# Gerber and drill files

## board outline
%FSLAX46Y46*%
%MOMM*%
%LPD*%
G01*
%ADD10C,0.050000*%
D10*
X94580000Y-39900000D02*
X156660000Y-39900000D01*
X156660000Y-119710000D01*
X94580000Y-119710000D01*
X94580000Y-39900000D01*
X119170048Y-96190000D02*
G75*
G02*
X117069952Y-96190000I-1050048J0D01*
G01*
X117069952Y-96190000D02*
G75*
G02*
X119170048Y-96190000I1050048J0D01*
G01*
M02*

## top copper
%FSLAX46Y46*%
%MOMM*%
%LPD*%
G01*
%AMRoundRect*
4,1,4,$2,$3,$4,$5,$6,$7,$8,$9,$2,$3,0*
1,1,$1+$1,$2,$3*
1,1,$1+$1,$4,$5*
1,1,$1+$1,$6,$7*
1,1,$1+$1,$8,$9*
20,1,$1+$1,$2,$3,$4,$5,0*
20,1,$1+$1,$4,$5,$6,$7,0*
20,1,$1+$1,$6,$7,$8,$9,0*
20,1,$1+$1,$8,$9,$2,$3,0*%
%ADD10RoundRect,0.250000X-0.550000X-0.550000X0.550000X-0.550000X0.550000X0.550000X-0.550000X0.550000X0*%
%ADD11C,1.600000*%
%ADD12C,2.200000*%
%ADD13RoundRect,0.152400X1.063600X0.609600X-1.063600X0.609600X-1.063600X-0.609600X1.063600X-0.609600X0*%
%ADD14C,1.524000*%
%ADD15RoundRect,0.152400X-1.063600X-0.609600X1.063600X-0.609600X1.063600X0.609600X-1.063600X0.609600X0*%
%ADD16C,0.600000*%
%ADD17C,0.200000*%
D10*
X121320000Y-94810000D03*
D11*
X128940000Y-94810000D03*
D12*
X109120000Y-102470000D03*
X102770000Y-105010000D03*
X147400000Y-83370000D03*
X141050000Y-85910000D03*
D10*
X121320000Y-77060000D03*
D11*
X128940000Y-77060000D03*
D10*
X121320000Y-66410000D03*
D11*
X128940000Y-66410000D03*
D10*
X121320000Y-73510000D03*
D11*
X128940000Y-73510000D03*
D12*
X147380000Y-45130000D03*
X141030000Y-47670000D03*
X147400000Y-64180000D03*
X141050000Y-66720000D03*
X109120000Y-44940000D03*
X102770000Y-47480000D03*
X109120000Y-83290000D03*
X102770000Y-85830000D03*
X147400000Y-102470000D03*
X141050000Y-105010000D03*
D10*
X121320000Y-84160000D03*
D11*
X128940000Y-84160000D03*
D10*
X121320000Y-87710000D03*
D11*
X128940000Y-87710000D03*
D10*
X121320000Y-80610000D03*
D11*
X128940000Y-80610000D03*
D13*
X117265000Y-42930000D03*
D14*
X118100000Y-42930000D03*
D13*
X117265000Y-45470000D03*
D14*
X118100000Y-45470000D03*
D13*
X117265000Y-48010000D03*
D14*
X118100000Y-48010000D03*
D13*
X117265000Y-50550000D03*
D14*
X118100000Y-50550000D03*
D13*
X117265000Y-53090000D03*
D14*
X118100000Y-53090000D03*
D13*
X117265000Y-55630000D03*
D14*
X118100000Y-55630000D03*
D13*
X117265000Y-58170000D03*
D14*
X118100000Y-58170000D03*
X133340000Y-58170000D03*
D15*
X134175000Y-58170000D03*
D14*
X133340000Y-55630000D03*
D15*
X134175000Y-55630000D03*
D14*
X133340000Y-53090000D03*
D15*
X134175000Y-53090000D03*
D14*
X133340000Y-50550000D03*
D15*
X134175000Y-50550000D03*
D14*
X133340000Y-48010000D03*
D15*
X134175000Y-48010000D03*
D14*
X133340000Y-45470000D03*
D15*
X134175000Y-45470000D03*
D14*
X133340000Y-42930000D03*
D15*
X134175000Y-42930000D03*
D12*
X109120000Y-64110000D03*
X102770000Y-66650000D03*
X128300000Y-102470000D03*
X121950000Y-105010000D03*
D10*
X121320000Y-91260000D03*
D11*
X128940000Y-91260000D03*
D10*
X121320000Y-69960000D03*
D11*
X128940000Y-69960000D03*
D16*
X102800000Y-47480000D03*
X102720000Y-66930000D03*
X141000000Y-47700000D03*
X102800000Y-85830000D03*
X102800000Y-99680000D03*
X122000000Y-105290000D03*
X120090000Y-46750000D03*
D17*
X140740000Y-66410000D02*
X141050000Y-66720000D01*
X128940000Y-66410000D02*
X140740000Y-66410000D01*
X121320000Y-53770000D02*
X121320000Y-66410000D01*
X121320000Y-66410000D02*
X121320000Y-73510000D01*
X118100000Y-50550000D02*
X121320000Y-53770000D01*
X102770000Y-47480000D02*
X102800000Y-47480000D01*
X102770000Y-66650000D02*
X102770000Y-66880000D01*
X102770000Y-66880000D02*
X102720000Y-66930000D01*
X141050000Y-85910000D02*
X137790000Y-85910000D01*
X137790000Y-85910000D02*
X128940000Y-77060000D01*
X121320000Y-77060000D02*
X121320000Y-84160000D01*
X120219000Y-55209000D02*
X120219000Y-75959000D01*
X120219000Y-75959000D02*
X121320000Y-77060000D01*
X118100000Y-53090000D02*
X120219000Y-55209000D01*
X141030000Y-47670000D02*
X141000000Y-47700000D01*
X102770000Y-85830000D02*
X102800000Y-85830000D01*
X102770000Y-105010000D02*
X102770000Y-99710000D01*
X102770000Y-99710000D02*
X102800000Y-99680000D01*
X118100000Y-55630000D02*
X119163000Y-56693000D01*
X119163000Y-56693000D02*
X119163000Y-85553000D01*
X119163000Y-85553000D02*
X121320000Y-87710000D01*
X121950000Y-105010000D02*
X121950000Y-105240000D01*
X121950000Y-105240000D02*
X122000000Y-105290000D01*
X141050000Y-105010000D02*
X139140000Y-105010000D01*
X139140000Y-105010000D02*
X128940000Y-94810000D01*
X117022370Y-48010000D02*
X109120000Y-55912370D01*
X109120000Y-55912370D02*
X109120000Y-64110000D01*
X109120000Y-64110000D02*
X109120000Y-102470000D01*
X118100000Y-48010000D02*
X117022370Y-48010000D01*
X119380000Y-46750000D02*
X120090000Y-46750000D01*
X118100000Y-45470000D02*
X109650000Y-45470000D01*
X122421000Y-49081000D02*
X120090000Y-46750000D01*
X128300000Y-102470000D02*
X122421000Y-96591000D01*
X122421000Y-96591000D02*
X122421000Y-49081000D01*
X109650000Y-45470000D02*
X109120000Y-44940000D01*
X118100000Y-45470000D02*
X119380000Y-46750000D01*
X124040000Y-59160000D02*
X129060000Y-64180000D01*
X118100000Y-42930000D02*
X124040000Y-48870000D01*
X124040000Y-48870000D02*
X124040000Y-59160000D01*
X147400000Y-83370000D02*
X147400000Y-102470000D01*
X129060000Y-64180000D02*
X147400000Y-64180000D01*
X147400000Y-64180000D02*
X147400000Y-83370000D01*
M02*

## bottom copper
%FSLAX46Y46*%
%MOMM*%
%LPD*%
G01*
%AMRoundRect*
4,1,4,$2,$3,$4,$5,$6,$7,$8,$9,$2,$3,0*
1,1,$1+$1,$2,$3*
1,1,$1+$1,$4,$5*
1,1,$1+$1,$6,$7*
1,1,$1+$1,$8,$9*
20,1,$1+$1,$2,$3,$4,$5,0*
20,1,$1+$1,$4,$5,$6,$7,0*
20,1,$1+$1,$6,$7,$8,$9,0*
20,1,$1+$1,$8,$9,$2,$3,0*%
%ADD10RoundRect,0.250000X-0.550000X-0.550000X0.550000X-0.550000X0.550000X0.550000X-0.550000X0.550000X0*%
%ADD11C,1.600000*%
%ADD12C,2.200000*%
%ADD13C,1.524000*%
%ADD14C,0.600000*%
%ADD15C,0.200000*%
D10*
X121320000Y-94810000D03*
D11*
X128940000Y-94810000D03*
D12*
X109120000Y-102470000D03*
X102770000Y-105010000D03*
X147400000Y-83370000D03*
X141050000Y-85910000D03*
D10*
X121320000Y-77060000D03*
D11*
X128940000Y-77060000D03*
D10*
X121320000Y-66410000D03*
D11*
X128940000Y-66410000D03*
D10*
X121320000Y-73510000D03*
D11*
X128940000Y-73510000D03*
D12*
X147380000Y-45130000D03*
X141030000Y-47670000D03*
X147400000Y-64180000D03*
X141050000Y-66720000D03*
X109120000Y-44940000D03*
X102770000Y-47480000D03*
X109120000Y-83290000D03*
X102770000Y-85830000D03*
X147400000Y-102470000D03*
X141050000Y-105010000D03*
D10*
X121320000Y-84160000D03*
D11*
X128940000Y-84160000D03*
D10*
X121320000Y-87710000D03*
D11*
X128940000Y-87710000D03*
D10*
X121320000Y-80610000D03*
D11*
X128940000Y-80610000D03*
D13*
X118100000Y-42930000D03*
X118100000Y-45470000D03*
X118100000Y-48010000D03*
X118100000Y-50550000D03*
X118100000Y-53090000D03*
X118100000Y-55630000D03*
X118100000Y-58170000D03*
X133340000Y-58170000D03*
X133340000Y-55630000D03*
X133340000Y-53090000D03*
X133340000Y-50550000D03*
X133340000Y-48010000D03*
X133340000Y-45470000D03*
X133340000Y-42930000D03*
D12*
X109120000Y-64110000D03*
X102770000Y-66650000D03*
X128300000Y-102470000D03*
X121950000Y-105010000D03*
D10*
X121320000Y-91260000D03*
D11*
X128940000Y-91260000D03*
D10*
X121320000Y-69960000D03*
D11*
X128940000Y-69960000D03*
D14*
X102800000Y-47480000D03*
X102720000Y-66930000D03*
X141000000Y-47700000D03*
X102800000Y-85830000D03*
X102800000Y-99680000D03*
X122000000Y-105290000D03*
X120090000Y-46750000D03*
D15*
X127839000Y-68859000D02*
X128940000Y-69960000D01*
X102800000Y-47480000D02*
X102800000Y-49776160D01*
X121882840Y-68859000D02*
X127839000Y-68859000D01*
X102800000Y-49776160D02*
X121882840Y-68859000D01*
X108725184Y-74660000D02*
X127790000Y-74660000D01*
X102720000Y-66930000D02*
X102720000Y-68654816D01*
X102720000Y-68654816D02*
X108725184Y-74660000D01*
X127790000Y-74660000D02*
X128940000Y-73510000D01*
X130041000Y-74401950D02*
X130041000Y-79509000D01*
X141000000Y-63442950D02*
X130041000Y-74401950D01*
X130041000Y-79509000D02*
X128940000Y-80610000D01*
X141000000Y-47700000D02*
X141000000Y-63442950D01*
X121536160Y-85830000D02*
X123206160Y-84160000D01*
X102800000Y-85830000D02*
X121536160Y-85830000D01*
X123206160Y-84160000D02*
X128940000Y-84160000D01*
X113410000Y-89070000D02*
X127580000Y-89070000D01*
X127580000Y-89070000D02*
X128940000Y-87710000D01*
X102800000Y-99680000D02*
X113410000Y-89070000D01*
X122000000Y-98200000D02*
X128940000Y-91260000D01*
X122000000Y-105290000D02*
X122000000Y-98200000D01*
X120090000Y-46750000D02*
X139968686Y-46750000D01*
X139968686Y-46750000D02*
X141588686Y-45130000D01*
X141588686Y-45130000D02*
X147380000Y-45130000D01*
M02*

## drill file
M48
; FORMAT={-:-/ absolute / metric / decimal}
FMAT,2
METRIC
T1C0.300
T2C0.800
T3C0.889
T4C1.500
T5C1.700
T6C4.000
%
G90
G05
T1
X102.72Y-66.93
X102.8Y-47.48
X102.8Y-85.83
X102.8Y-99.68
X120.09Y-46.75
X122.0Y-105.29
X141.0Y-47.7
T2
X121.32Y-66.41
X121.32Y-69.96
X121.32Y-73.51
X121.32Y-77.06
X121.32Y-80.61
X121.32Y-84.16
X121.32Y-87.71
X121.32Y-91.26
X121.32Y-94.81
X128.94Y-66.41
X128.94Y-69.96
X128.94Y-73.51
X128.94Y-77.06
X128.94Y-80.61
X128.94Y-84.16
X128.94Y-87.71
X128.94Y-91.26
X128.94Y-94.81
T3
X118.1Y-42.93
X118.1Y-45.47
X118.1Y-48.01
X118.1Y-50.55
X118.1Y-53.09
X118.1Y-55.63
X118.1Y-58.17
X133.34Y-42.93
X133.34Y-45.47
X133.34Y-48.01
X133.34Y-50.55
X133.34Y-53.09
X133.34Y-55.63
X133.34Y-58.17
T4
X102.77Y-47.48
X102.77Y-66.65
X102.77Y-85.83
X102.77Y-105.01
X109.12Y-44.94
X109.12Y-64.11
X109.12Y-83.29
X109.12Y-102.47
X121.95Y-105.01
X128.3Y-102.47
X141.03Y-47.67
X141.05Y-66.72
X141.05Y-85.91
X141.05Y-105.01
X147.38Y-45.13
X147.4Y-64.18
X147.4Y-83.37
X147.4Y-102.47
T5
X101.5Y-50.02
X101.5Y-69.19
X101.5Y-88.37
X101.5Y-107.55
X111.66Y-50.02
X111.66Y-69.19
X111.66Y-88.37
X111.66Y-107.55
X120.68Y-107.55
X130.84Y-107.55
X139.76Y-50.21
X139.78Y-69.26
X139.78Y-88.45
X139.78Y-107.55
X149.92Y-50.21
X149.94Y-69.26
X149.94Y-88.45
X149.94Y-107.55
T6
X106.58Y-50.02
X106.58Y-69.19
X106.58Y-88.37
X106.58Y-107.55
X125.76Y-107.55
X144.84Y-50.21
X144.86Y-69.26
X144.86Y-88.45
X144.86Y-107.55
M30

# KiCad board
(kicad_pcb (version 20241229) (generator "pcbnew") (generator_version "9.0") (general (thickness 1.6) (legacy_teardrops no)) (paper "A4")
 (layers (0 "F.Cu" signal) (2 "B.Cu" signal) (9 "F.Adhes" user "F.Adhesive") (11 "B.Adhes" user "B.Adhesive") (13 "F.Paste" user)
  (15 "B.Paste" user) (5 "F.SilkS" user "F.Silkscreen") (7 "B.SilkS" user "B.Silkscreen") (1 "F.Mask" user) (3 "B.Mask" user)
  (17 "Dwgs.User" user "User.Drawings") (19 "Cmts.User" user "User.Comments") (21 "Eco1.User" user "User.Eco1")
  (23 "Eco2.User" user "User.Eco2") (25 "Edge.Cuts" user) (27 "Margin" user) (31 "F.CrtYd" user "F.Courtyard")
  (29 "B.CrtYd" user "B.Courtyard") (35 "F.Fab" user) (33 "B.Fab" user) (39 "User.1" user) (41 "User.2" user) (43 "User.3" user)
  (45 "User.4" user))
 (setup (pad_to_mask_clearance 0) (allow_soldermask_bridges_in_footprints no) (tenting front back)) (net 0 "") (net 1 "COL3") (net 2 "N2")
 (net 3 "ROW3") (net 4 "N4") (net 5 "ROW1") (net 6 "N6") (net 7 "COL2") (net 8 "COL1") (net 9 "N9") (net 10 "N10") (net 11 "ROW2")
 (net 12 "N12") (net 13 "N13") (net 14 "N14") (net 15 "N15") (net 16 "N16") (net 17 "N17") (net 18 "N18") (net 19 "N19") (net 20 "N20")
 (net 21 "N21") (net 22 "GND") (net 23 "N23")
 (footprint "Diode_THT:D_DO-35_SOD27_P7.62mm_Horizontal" (layer "F.Cu") (at 121.32 94.81)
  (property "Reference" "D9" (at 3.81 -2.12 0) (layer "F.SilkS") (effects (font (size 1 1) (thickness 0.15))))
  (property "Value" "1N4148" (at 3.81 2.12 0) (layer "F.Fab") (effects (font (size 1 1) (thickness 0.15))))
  (pad "1" thru_hole roundrect (at 0 0) (size 1.6 1.6) (drill 0.8) (layers "*.Cu" "*.Mask") (remove_unused_layers no)
   (roundrect_rratio 0.15625) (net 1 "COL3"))
  (pad "2" thru_hole circle (at 7.62 0) (size 1.6 1.6) (drill 0.8) (layers "*.Cu" "*.Mask") (remove_unused_layers no) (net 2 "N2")))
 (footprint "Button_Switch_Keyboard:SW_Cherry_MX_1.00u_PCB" (layer "F.Cu") (at 109.12 102.47)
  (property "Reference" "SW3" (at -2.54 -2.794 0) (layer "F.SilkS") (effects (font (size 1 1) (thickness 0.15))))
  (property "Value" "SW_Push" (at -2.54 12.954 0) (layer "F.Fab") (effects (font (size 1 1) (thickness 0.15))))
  (pad "" np_thru_hole circle (at -7.62 5.08) (size 1.7 1.7) (drill 1.7) (layers "*.Cu" "*.Mask"))
  (pad "" np_thru_hole circle (at -2.54 5.08) (size 4 4) (drill 4) (layers "*.Cu" "*.Mask"))
  (pad "" np_thru_hole circle (at 2.54 5.08) (size 1.7 1.7) (drill 1.7) (layers "*.Cu" "*.Mask"))
  (pad "1" thru_hole circle (at 0 0) (size 2.2 2.2) (drill 1.5) (layers "*.Cu" "*.Mask") (remove_unused_layers no) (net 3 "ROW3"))
  (pad "2" thru_hole circle (at -6.35 2.54) (size 2.2 2.2) (drill 1.5) (layers "*.Cu" "*.Mask") (remove_unused_layers no) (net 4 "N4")))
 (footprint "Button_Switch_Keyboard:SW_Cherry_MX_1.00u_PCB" (layer "F.Cu") (at 147.4 83.37)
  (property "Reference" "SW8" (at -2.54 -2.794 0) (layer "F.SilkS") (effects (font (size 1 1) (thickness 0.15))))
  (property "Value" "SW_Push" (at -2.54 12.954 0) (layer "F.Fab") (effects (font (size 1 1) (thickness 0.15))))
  (pad "" np_thru_hole circle (at -7.62 5.08) (size 1.7 1.7) (drill 1.7) (layers "*.Cu" "*.Mask"))
  (pad "" np_thru_hole circle (at -2.54 5.08) (size 4 4) (drill 4) (layers "*.Cu" "*.Mask"))
  (pad "" np_thru_hole circle (at 2.54 5.08) (size 1.7 1.7) (drill 1.7) (layers "*.Cu" "*.Mask"))
  (pad "1" thru_hole circle (at 0 0) (size 2.2 2.2) (drill 1.5) (layers "*.Cu" "*.Mask") (remove_unused_layers no) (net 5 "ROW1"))
  (pad "2" thru_hole circle (at -6.35 2.54) (size 2.2 2.2) (drill 1.5) (layers "*.Cu" "*.Mask") (remove_unused_layers no) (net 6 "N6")))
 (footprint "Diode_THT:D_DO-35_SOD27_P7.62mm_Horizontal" (layer "F.Cu") (at 121.32 77.06)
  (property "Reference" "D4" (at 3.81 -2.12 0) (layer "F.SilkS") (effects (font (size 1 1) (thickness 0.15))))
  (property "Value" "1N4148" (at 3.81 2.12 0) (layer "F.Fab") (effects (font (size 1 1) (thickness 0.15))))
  (pad "1" thru_hole roundrect (at 0 0) (size 1.6 1.6) (drill 0.8) (layers "*.Cu" "*.Mask") (remove_unused_layers no)
   (roundrect_rratio 0.15625) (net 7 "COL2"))
  (pad "2" thru_hole circle (at 7.62 0) (size 1.6 1.6) (drill 0.8) (layers "*.Cu" "*.Mask") (remove_unused_layers no) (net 6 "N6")))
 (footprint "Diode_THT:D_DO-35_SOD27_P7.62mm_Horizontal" (layer "F.Cu") (at 121.32 66.41)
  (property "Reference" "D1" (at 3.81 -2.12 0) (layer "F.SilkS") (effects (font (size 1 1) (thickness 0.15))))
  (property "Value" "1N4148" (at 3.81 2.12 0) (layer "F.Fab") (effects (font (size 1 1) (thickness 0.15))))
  (pad "1" thru_hole roundrect (at 0 0) (size 1.6 1.6) (drill 0.8) (layers "*.Cu" "*.Mask") (remove_unused_layers no)
   (roundrect_rratio 0.15625) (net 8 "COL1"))
  (pad "2" thru_hole circle (at 7.62 0) (size 1.6 1.6) (drill 0.8) (layers "*.Cu" "*.Mask") (remove_unused_layers no) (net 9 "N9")))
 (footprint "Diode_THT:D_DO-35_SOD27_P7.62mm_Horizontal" (layer "F.Cu") (at 121.32 73.51)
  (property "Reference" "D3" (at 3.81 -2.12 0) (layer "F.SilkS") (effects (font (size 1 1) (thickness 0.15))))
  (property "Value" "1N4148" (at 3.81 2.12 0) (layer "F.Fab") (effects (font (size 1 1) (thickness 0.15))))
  (pad "1" thru_hole roundrect (at 0 0) (size 1.6 1.6) (drill 0.8) (layers "*.Cu" "*.Mask") (remove_unused_layers no)
   (roundrect_rratio 0.15625) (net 8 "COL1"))
  (pad "2" thru_hole circle (at 7.62 0) (size 1.6 1.6) (drill 0.8) (layers "*.Cu" "*.Mask") (remove_unused_layers no) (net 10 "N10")))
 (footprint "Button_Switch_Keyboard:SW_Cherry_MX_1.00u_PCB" (layer "F.Cu") (at 147.38 45.13)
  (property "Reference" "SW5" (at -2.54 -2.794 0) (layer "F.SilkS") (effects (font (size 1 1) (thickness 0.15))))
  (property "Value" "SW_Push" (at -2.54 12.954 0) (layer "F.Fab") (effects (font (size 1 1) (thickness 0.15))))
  (pad "" np_thru_hole circle (at -7.62 5.08) (size 1.7 1.7) (drill 1.7) (layers "*.Cu" "*.Mask"))
  (pad "" np_thru_hole circle (at -2.54 5.08) (size 4 4) (drill 4) (layers "*.Cu" "*.Mask"))
  (pad "" np_thru_hole circle (at 2.54 5.08) (size 1.7 1.7) (drill 1.7) (layers "*.Cu" "*.Mask"))
  (pad "1" thru_hole circle (at 0 0) (size 2.2 2.2) (drill 1.5) (layers "*.Cu" "*.Mask") (remove_unused_layers no) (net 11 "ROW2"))
  (pad "2" thru_hole circle (at -6.35 2.54) (size 2.2 2.2) (drill 1.5) (layers "*.Cu" "*.Mask") (remove_unused_layers no) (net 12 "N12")))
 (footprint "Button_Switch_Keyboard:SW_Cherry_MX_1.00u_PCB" (layer "F.Cu") (at 147.4 64.18)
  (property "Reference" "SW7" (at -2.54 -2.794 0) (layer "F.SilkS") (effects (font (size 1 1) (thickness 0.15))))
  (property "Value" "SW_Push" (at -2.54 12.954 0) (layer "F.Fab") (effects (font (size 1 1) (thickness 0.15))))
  (pad "" np_thru_hole circle (at -7.62 5.08) (size 1.7 1.7) (drill 1.7) (layers "*.Cu" "*.Mask"))
  (pad "" np_thru_hole circle (at -2.54 5.08) (size 4 4) (drill 4) (layers "*.Cu" "*.Mask"))
  (pad "" np_thru_hole circle (at 2.54 5.08) (size 1.7 1.7) (drill 1.7) (layers "*.Cu" "*.Mask"))
  (pad "1" thru_hole circle (at 0 0) (size 2.2 2.2) (drill 1.5) (layers "*.Cu" "*.Mask") (remove_unused_layers no) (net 5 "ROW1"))
  (pad "2" thru_hole circle (at -6.35 2.54) (size 2.2 2.2) (drill 1.5) (layers "*.Cu" "*.Mask") (remove_unused_layers no) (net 9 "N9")))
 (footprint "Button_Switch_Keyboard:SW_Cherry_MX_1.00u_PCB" (layer "F.Cu") (at 109.12 44.94)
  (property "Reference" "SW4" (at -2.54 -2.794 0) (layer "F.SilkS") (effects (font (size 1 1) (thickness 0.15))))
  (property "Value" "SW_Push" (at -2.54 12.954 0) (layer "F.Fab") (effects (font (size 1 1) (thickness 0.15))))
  (pad "" np_thru_hole circle (at -7.62 5.08) (size 1.7 1.7) (drill 1.7) (layers "*.Cu" "*.Mask"))
  (pad "" np_thru_hole circle (at -2.54 5.08) (size 4 4) (drill 4) (layers "*.Cu" "*.Mask"))
  (pad "" np_thru_hole circle (at 2.54 5.08) (size 1.7 1.7) (drill 1.7) (layers "*.Cu" "*.Mask"))
  (pad "1" thru_hole circle (at 0 0) (size 2.2 2.2) (drill 1.5) (layers "*.Cu" "*.Mask") (remove_unused_layers no) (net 11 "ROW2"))
  (pad "2" thru_hole circle (at -6.35 2.54) (size 2.2 2.2) (drill 1.5) (layers "*.Cu" "*.Mask") (remove_unused_layers no) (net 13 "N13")))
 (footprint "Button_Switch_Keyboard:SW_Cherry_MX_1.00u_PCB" (layer "F.Cu") (at 109.12 83.29)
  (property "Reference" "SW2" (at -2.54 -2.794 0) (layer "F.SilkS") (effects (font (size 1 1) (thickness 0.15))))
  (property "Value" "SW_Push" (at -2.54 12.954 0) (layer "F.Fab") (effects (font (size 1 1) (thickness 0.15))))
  (pad "" np_thru_hole circle (at -7.62 5.08) (size 1.7 1.7) (drill 1.7) (layers "*.Cu" "*.Mask"))
  (pad "" np_thru_hole circle (at -2.54 5.08) (size 4 4) (drill 4) (layers "*.Cu" "*.Mask"))
  (pad "" np_thru_hole circle (at 2.54 5.08) (size 1.7 1.7) (drill 1.7) (layers "*.Cu" "*.Mask"))
  (pad "1" thru_hole circle (at 0 0) (size 2.2 2.2) (drill 1.5) (layers "*.Cu" "*.Mask") (remove_unused_layers no) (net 3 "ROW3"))
  (pad "2" thru_hole circle (at -6.35 2.54) (size 2.2 2.2) (drill 1.5) (layers "*.Cu" "*.Mask") (remove_unused_layers no) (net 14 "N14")))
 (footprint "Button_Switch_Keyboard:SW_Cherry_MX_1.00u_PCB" (layer "F.Cu") (at 147.4 102.47)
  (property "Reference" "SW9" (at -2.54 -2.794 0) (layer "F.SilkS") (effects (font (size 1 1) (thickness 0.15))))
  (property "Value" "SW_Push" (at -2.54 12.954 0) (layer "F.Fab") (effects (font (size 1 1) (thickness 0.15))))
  (pad "" np_thru_hole circle (at -7.62 5.08) (size 1.7 1.7) (drill 1.7) (layers "*.Cu" "*.Mask"))
  (pad "" np_thru_hole circle (at -2.54 5.08) (size 4 4) (drill 4) (layers "*.Cu" "*.Mask"))
  (pad "" np_thru_hole circle (at 2.54 5.08) (size 1.7 1.7) (drill 1.7) (layers "*.Cu" "*.Mask"))
  (pad "1" thru_hole circle (at 0 0) (size 2.2 2.2) (drill 1.5) (layers "*.Cu" "*.Mask") (remove_unused_layers no) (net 5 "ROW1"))
  (pad "2" thru_hole circle (at -6.35 2.54) (size 2.2 2.2) (drill 1.5) (layers "*.Cu" "*.Mask") (remove_unused_layers no) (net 2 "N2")))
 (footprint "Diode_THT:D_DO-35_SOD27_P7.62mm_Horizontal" (layer "F.Cu") (at 121.32 84.16)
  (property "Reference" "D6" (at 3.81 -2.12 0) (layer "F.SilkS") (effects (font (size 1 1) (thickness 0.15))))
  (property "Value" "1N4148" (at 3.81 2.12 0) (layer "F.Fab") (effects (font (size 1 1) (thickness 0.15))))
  (pad "1" thru_hole roundrect (at 0 0) (size 1.6 1.6) (drill 0.8) (layers "*.Cu" "*.Mask") (remove_unused_layers no)
   (roundrect_rratio 0.15625) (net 7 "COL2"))
  (pad "2" thru_hole circle (at 7.62 0) (size 1.6 1.6) (drill 0.8) (layers "*.Cu" "*.Mask") (remove_unused_layers no) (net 14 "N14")))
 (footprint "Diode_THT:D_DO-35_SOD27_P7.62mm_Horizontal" (layer "F.Cu") (at 121.32 87.71)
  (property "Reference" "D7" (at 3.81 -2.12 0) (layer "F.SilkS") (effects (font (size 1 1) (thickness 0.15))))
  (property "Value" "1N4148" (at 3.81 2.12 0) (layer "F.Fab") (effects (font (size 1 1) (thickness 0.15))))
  (pad "1" thru_hole roundrect (at 0 0) (size 1.6 1.6) (drill 0.8) (layers "*.Cu" "*.Mask") (remove_unused_layers no)
   (roundrect_rratio 0.15625) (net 1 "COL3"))
  (pad "2" thru_hole circle (at 7.62 0) (size 1.6 1.6) (drill 0.8) (layers "*.Cu" "*.Mask") (remove_unused_layers no) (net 4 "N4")))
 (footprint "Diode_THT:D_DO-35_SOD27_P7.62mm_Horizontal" (layer "F.Cu") (at 121.32 80.61)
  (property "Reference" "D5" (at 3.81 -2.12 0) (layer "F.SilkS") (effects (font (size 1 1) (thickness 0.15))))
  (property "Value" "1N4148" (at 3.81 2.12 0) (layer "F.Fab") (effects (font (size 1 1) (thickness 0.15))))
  (pad "1" thru_hole roundrect (at 0 0) (size 1.6 1.6) (drill 0.8) (layers "*.Cu" "*.Mask") (remove_unused_layers no)
   (roundrect_rratio 0.15625) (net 7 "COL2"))
  (pad "2" thru_hole circle (at 7.62 0) (size 1.6 1.6) (drill 0.8) (layers "*.Cu" "*.Mask") (remove_unused_layers no) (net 12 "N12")))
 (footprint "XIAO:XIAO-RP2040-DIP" (layer "F.Cu") (at 125.72 50.55)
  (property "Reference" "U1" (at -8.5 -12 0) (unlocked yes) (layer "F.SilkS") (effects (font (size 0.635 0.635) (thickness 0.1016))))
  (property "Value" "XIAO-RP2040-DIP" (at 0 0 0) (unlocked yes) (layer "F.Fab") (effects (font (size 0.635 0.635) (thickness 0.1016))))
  (pad "1" smd roundrect (at -8.455 -7.62 180) (size 2.432 1.524) (layers "F.Cu" "F.Mask") (roundrect_rratio 0.1) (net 5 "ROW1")
   (thermal_bridge_angle 45))
  (pad "1" thru_hole circle (at -7.62 -7.62 180) (size 1.524 1.524) (drill 0.889) (layers "*.Cu" "*.Mask") (remove_unused_layers no)
   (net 5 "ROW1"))
  (pad "2" smd roundrect (at -8.455 -5.08 180) (size 2.432 1.524) (layers "F.Cu" "F.Mask") (roundrect_rratio 0.1) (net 11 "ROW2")
   (thermal_bridge_angle 45))
  (pad "2" thru_hole circle (at -7.62 -5.08 180) (size 1.524 1.524) (drill 0.889) (layers "*.Cu" "*.Mask") (remove_unused_layers no)
   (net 11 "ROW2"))
  (pad "3" smd roundrect (at -8.455 -2.54 180) (size 2.432 1.524) (layers "F.Cu" "F.Mask") (roundrect_rratio 0.1) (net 3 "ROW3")
   (thermal_bridge_angle 45))
  (pad "3" thru_hole circle (at -7.62 -2.54 180) (size 1.524 1.524) (drill 0.889) (layers "*.Cu" "*.Mask") (remove_unused_layers no)
   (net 3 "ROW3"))
  (pad "4" smd roundrect (at -8.455 0 180) (size 2.432 1.524) (layers "F.Cu" "F.Mask") (roundrect_rratio 0.1) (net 8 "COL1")
   (thermal_bridge_angle 45))
  (pad "4" thru_hole circle (at -7.62 0 180) (size 1.524 1.524) (drill 0.889) (layers "*.Cu" "*.Mask") (remove_unused_layers no)
   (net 8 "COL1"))
  (pad "5" smd roundrect (at -8.455 2.54 180) (size 2.432 1.524) (layers "F.Cu" "F.Mask") (roundrect_rratio 0.1) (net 7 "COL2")
   (thermal_bridge_angle 45))
  (pad "5" thru_hole circle (at -7.62 2.54 180) (size 1.524 1.524) (drill 0.889) (layers "*.Cu" "*.Mask") (remove_unused_layers no)
   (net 7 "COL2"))
  (pad "6" smd roundrect (at -8.455 5.08 180) (size 2.432 1.524) (layers "F.Cu" "F.Mask") (roundrect_rratio 0.1) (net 1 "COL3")
   (thermal_bridge_angle 45))
  (pad "6" thru_hole circle (at -7.62 5.08 180) (size 1.524 1.524) (drill 0.889) (layers "*.Cu" "*.Mask") (remove_unused_layers no)
   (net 1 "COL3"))
  (pad "7" smd roundrect (at -8.455 7.62 180) (size 2.432 1.524) (layers "F.Cu" "F.Mask") (roundrect_rratio 0.1) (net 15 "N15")
   (thermal_bridge_angle 45))
  (pad "7" thru_hole circle (at -7.62 7.62 180) (size 1.524 1.524) (drill 0.889) (layers "*.Cu" "*.Mask") (remove_unused_layers no)
   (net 15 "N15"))
  (pad "8" thru_hole circle (at 7.62 7.62) (size 1.524 1.524) (drill 0.889) (layers "*.Cu" "*.Mask") (remove_unused_layers no)
   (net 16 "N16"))
  (pad "8" smd roundrect (at 8.455 7.62) (size 2.432 1.524) (layers "F.Cu" "F.Mask") (roundrect_rratio 0.1) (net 16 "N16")
   (thermal_bridge_angle 45))
  (pad "9" thru_hole circle (at 7.62 5.08) (size 1.524 1.524) (drill 0.889) (layers "*.Cu" "*.Mask") (remove_unused_layers no)
   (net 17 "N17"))
  (pad "9" smd roundrect (at 8.455 5.08) (size 2.432 1.524) (layers "F.Cu" "F.Mask") (roundrect_rratio 0.1) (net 17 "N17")
   (thermal_bridge_angle 45))
  (pad "10" thru_hole circle (at 7.62 2.54) (size 1.524 1.524) (drill 0.889) (layers "*.Cu" "*.Mask") (remove_unused_layers no)
   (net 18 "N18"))
  (pad "10" smd roundrect (at 8.455 2.54) (size 2.432 1.524) (layers "F.Cu" "F.Mask") (roundrect_rratio 0.1) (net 18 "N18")
   (thermal_bridge_angle 45))
  (pad "11" thru_hole circle (at 7.62 0) (size 1.524 1.524) (drill 0.889) (layers "*.Cu" "*.Mask") (remove_unused_layers no) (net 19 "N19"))
  (pad "11" smd roundrect (at 8.455 0) (size 2.432 1.524) (layers "F.Cu" "F.Mask") (roundrect_rratio 0.1) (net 19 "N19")
   (thermal_bridge_angle 45))
  (pad "12" thru_hole circle (at 7.62 -2.54) (size 1.524 1.524) (drill 0.889) (layers "*.Cu" "*.Mask") (remove_unused_layers no)
   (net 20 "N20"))
  (pad "12" smd roundrect (at 8.455 -2.54) (size 2.432 1.524) (layers "F.Cu" "F.Mask") (roundrect_rratio 0.1) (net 20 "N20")
   (thermal_bridge_angle 45))
  (pad "13" thru_hole circle (at 7.62 -5.08) (size 1.524 1.524) (drill 0.889) (layers "*.Cu" "*.Mask") (remove_unused_layers no)
   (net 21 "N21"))
  (pad "13" smd roundrect (at 8.455 -5.08) (size 2.432 1.524) (layers "F.Cu" "F.Mask") (roundrect_rratio 0.1) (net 21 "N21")
   (thermal_bridge_angle 45))
  (pad "14" thru_hole circle (at 7.62 -7.62) (size 1.524 1.524) (drill 0.889) (layers "*.Cu" "*.Mask") (remove_unused_layers no)
   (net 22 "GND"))
  (pad "14" smd roundrect (at 8.455 -7.62) (size 2.432 1.524) (layers "F.Cu" "F.Mask") (roundrect_rratio 0.1) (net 22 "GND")
   (thermal_bridge_angle 45)))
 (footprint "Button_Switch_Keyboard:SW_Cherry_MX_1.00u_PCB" (layer "F.Cu") (at 109.12 64.11)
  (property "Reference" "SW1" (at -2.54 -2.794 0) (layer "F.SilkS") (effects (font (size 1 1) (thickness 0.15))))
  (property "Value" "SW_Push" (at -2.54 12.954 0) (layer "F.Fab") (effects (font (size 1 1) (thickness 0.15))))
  (pad "" np_thru_hole circle (at -7.62 5.08) (size 1.7 1.7) (drill 1.7) (layers "*.Cu" "*.Mask"))
  (pad "" np_thru_hole circle (at -2.54 5.08) (size 4 4) (drill 4) (layers "*.Cu" "*.Mask"))
  (pad "" np_thru_hole circle (at 2.54 5.08) (size 1.7 1.7) (drill 1.7) (layers "*.Cu" "*.Mask"))
  (pad "1" thru_hole circle (at 0 0) (size 2.2 2.2) (drill 1.5) (layers "*.Cu" "*.Mask") (remove_unused_layers no) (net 3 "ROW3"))
  (pad "2" thru_hole circle (at -6.35 2.54) (size 2.2 2.2) (drill 1.5) (layers "*.Cu" "*.Mask") (remove_unused_layers no) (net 10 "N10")))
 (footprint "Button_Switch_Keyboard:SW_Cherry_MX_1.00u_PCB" (layer "F.Cu") (at 128.3 102.47)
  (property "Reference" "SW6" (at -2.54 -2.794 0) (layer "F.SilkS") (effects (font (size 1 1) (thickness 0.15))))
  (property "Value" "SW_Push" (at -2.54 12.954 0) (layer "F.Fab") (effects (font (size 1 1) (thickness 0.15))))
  (pad "" np_thru_hole circle (at -7.62 5.08) (size 1.7 1.7) (drill 1.7) (layers "*.Cu" "*.Mask"))
  (pad "" np_thru_hole circle (at -2.54 5.08) (size 4 4) (drill 4) (layers "*.Cu" "*.Mask"))
  (pad "" np_thru_hole circle (at 2.54 5.08) (size 1.7 1.7) (drill 1.7) (layers "*.Cu" "*.Mask"))
  (pad "1" thru_hole circle (at 0 0) (size 2.2 2.2) (drill 1.5) (layers "*.Cu" "*.Mask") (remove_unused_layers no) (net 11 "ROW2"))
  (pad "2" thru_hole circle (at -6.35 2.54) (size 2.2 2.2) (drill 1.5) (layers "*.Cu" "*.Mask") (remove_unused_layers no) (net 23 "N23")))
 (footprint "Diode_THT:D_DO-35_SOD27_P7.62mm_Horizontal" (layer "F.Cu") (at 121.32 91.26)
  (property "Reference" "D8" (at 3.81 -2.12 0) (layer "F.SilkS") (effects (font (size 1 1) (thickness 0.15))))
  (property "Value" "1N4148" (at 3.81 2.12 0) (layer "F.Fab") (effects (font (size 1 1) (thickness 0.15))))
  (pad "1" thru_hole roundrect (at 0 0) (size 1.6 1.6) (drill 0.8) (layers "*.Cu" "*.Mask") (remove_unused_layers no)
   (roundrect_rratio 0.15625) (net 1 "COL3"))
  (pad "2" thru_hole circle (at 7.62 0) (size 1.6 1.6) (drill 0.8) (layers "*.Cu" "*.Mask") (remove_unused_layers no) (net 23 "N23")))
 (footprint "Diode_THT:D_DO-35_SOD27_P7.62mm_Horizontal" (layer "F.Cu") (at 121.32 69.96)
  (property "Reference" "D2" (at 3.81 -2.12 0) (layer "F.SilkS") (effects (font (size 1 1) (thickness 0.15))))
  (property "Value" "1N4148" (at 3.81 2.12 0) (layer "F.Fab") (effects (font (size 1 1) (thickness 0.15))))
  (pad "1" thru_hole roundrect (at 0 0) (size 1.6 1.6) (drill 0.8) (layers "*.Cu" "*.Mask") (remove_unused_layers no)
   (roundrect_rratio 0.15625) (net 8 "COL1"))
  (pad "2" thru_hole circle (at 7.62 0) (size 1.6 1.6) (drill 0.8) (layers "*.Cu" "*.Mask") (remove_unused_layers no) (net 13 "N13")))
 (gr_rect (start 94.58 39.9) (end 156.66 119.71) (stroke (width 0.05) (type default)) (fill no) (layer "Edge.Cuts"))
 (gr_circle (center 118.12 96.19) (end 117.07 96.18) (stroke (width 0.05) (type default)) (fill no) (layer "Edge.Cuts"))
 (segment (start 140.74 66.41) (end 141.05 66.72) (width 0.2) (layer "F.Cu") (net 9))
 (segment (start 128.94 66.41) (end 140.74 66.41) (width 0.2) (layer "F.Cu") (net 9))
 (segment (start 121.32 53.77) (end 121.32 66.41) (width 0.2) (layer "F.Cu") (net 8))
 (segment (start 121.32 66.41) (end 121.32 73.51) (width 0.2) (layer "F.Cu") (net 8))
 (segment (start 118.1 50.55) (end 121.32 53.77) (width 0.2) (layer "F.Cu") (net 8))
 (segment (start 102.77 47.48) (end 102.8 47.48) (width 0.2) (layer "F.Cu") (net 13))
 (via (at 102.8 47.48) (size 0.6) (drill 0.3) (layers "F.Cu" "B.Cu") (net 13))
 (segment (start 127.839 68.859) (end 128.94 69.96) (width 0.2) (layer "B.Cu") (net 13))
 (segment (start 102.8 47.48) (end 102.8 49.77616) (width 0.2) (layer "B.Cu") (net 13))
 (segment (start 121.88284 68.859) (end 127.839 68.859) (width 0.2) (layer "B.Cu") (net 13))
 (segment (start 102.8 49.77616) (end 121.88284 68.859) (width 0.2) (layer "B.Cu") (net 13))
 (segment (start 102.77 66.65) (end 102.77 66.88) (width 0.2) (layer "F.Cu") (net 10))
 (segment (start 102.77 66.88) (end 102.72 66.93) (width 0.2) (layer "F.Cu") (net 10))
 (via (at 102.72 66.93) (size 0.6) (drill 0.3) (layers "F.Cu" "B.Cu") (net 10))
 (segment (start 108.725184 74.66) (end 127.79 74.66) (width 0.2) (layer "B.Cu") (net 10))
 (segment (start 102.72 66.93) (end 102.72 68.654816) (width 0.2) (layer "B.Cu") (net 10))
 (segment (start 102.72 68.654816) (end 108.725184 74.66) (width 0.2) (layer "B.Cu") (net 10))
 (segment (start 127.79 74.66) (end 128.94 73.51) (width 0.2) (layer "B.Cu") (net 10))
 (segment (start 141.05 85.91) (end 137.79 85.91) (width 0.2) (layer "F.Cu") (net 6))
 (segment (start 137.79 85.91) (end 128.94 77.06) (width 0.2) (layer "F.Cu") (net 6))
 (segment (start 121.32 77.06) (end 121.32 84.16) (width 0.2) (layer "F.Cu") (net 7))
 (segment (start 120.219 55.209) (end 120.219 75.959) (width 0.2) (layer "F.Cu") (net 7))
 (segment (start 120.219 75.959) (end 121.32 77.06) (width 0.2) (layer "F.Cu") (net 7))
 (segment (start 118.1 53.09) (end 120.219 55.209) (width 0.2) (layer "F.Cu") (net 7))
 (segment (start 141.03 47.67) (end 141 47.7) (width 0.2) (layer "F.Cu") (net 12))
 (via (at 141 47.7) (size 0.6) (drill 0.3) (layers "F.Cu" "B.Cu") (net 12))
 (segment (start 130.041 74.40195) (end 130.041 79.509) (width 0.2) (layer "B.Cu") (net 12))
 (segment (start 141 63.44295) (end 130.041 74.40195) (width 0.2) (layer "B.Cu") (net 12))
 (segment (start 130.041 79.509) (end 128.94 80.61) (width 0.2) (layer "B.Cu") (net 12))
 (segment (start 141 47.7) (end 141 63.44295) (width 0.2) (layer "B.Cu") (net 12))
 (segment (start 102.77 85.83) (end 102.8 85.83) (width 0.2) (layer "F.Cu") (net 14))
 (via (at 102.8 85.83) (size 0.6) (drill 0.3) (layers "F.Cu" "B.Cu") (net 14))
 (segment (start 121.53616 85.83) (end 123.20616 84.16) (width 0.2) (layer "B.Cu") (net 14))
 (segment (start 102.8 85.83) (end 121.53616 85.83) (width 0.2) (layer "B.Cu") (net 14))
 (segment (start 123.20616 84.16) (end 128.94 84.16) (width 0.2) (layer "B.Cu") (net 14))
 (segment (start 102.77 105.01) (end 102.77 99.71) (width 0.2) (layer "F.Cu") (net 4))
 (segment (start 102.77 99.71) (end 102.8 99.68) (width 0.2) (layer "F.Cu") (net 4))
 (via (at 102.8 99.68) (size 0.6) (drill 0.3) (layers "F.Cu" "B.Cu") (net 4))
 (segment (start 113.41 89.07) (end 127.58 89.07) (width 0.2) (layer "B.Cu") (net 4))
 (segment (start 127.58 89.07) (end 128.94 87.71) (width 0.2) (layer "B.Cu") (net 4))
 (segment (start 102.8 99.68) (end 113.41 89.07) (width 0.2) (layer "B.Cu") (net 4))
 (segment (start 118.1 55.63) (end 119.163 56.693) (width 0.2) (layer "F.Cu") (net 1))
 (segment (start 119.163 56.693) (end 119.163 85.553) (width 0.2) (layer "F.Cu") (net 1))
 (segment (start 119.163 85.553) (end 121.32 87.71) (width 0.2) (layer "F.Cu") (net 1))
 (segment (start 121.95 105.01) (end 121.95 105.24) (width 0.2) (layer "F.Cu") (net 23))
 (segment (start 121.95 105.24) (end 122 105.29) (width 0.2) (layer "F.Cu") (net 23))
 (via (at 122 105.29) (size 0.6) (drill 0.3) (layers "F.Cu" "B.Cu") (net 23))
 (segment (start 122 98.2) (end 128.94 91.26) (width 0.2) (layer "B.Cu") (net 23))
 (segment (start 122 105.29) (end 122 98.2) (width 0.2) (layer "B.Cu") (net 23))
 (segment (start 141.05 105.01) (end 139.14 105.01) (width 0.2) (layer "F.Cu") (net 2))
 (segment (start 139.14 105.01) (end 128.94 94.81) (width 0.2) (layer "F.Cu") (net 2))
 (segment (start 117.02237 48.01) (end 109.12 55.91237) (width 0.2) (layer "F.Cu") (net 3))
 (segment (start 109.12 55.91237) (end 109.12 64.11) (width 0.2) (layer "F.Cu") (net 3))
 (segment (start 109.12 64.11) (end 109.12 102.47) (width 0.2) (layer "F.Cu") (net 3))
 (segment (start 118.1 48.01) (end 117.02237 48.01) (width 0.2) (layer "F.Cu") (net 3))
 (segment (start 119.38 46.75) (end 120.09 46.75) (width 0.2) (layer "F.Cu") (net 11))
 (segment (start 118.1 45.47) (end 109.65 45.47) (width 0.2) (layer "F.Cu") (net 11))
 (segment (start 122.421 49.081) (end 120.09 46.75) (width 0.2) (layer "F.Cu") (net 11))
 (segment (start 128.3 102.47) (end 122.421 96.591) (width 0.2) (layer "F.Cu") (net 11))
 (segment (start 122.421 96.591) (end 122.421 49.081) (width 0.2) (layer "F.Cu") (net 11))
 (segment (start 109.65 45.47) (end 109.12 44.94) (width 0.2) (layer "F.Cu") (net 11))
 (segment (start 118.1 45.47) (end 119.38 46.75) (width 0.2) (layer "F.Cu") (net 11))
 (via (at 120.09 46.75) (size 0.6) (drill 0.3) (layers "F.Cu" "B.Cu") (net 11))
 (segment (start 120.09 46.75) (end 139.968686 46.75) (width 0.2) (layer "B.Cu") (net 11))
 (segment (start 139.968686 46.75) (end 141.588686 45.13) (width 0.2) (layer "B.Cu") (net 11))
 (segment (start 141.588686 45.13) (end 147.38 45.13) (width 0.2) (layer "B.Cu") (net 11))
 (segment (start 124.04 59.16) (end 129.06 64.18) (width 0.2) (layer "F.Cu") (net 5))
 (segment (start 118.1 42.93) (end 124.04 48.87) (width 0.2) (layer "F.Cu") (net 5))
 (segment (start 124.04 48.87) (end 124.04 59.16) (width 0.2) (layer "F.Cu") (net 5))
 (segment (start 147.4 83.37) (end 147.4 102.47) (width 0.2) (layer "F.Cu") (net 5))
 (segment (start 129.06 64.18) (end 147.4 64.18) (width 0.2) (layer "F.Cu") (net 5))
 (segment (start 147.4 64.18) (end 147.4 83.37) (width 0.2) (layer "F.Cu") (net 5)))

